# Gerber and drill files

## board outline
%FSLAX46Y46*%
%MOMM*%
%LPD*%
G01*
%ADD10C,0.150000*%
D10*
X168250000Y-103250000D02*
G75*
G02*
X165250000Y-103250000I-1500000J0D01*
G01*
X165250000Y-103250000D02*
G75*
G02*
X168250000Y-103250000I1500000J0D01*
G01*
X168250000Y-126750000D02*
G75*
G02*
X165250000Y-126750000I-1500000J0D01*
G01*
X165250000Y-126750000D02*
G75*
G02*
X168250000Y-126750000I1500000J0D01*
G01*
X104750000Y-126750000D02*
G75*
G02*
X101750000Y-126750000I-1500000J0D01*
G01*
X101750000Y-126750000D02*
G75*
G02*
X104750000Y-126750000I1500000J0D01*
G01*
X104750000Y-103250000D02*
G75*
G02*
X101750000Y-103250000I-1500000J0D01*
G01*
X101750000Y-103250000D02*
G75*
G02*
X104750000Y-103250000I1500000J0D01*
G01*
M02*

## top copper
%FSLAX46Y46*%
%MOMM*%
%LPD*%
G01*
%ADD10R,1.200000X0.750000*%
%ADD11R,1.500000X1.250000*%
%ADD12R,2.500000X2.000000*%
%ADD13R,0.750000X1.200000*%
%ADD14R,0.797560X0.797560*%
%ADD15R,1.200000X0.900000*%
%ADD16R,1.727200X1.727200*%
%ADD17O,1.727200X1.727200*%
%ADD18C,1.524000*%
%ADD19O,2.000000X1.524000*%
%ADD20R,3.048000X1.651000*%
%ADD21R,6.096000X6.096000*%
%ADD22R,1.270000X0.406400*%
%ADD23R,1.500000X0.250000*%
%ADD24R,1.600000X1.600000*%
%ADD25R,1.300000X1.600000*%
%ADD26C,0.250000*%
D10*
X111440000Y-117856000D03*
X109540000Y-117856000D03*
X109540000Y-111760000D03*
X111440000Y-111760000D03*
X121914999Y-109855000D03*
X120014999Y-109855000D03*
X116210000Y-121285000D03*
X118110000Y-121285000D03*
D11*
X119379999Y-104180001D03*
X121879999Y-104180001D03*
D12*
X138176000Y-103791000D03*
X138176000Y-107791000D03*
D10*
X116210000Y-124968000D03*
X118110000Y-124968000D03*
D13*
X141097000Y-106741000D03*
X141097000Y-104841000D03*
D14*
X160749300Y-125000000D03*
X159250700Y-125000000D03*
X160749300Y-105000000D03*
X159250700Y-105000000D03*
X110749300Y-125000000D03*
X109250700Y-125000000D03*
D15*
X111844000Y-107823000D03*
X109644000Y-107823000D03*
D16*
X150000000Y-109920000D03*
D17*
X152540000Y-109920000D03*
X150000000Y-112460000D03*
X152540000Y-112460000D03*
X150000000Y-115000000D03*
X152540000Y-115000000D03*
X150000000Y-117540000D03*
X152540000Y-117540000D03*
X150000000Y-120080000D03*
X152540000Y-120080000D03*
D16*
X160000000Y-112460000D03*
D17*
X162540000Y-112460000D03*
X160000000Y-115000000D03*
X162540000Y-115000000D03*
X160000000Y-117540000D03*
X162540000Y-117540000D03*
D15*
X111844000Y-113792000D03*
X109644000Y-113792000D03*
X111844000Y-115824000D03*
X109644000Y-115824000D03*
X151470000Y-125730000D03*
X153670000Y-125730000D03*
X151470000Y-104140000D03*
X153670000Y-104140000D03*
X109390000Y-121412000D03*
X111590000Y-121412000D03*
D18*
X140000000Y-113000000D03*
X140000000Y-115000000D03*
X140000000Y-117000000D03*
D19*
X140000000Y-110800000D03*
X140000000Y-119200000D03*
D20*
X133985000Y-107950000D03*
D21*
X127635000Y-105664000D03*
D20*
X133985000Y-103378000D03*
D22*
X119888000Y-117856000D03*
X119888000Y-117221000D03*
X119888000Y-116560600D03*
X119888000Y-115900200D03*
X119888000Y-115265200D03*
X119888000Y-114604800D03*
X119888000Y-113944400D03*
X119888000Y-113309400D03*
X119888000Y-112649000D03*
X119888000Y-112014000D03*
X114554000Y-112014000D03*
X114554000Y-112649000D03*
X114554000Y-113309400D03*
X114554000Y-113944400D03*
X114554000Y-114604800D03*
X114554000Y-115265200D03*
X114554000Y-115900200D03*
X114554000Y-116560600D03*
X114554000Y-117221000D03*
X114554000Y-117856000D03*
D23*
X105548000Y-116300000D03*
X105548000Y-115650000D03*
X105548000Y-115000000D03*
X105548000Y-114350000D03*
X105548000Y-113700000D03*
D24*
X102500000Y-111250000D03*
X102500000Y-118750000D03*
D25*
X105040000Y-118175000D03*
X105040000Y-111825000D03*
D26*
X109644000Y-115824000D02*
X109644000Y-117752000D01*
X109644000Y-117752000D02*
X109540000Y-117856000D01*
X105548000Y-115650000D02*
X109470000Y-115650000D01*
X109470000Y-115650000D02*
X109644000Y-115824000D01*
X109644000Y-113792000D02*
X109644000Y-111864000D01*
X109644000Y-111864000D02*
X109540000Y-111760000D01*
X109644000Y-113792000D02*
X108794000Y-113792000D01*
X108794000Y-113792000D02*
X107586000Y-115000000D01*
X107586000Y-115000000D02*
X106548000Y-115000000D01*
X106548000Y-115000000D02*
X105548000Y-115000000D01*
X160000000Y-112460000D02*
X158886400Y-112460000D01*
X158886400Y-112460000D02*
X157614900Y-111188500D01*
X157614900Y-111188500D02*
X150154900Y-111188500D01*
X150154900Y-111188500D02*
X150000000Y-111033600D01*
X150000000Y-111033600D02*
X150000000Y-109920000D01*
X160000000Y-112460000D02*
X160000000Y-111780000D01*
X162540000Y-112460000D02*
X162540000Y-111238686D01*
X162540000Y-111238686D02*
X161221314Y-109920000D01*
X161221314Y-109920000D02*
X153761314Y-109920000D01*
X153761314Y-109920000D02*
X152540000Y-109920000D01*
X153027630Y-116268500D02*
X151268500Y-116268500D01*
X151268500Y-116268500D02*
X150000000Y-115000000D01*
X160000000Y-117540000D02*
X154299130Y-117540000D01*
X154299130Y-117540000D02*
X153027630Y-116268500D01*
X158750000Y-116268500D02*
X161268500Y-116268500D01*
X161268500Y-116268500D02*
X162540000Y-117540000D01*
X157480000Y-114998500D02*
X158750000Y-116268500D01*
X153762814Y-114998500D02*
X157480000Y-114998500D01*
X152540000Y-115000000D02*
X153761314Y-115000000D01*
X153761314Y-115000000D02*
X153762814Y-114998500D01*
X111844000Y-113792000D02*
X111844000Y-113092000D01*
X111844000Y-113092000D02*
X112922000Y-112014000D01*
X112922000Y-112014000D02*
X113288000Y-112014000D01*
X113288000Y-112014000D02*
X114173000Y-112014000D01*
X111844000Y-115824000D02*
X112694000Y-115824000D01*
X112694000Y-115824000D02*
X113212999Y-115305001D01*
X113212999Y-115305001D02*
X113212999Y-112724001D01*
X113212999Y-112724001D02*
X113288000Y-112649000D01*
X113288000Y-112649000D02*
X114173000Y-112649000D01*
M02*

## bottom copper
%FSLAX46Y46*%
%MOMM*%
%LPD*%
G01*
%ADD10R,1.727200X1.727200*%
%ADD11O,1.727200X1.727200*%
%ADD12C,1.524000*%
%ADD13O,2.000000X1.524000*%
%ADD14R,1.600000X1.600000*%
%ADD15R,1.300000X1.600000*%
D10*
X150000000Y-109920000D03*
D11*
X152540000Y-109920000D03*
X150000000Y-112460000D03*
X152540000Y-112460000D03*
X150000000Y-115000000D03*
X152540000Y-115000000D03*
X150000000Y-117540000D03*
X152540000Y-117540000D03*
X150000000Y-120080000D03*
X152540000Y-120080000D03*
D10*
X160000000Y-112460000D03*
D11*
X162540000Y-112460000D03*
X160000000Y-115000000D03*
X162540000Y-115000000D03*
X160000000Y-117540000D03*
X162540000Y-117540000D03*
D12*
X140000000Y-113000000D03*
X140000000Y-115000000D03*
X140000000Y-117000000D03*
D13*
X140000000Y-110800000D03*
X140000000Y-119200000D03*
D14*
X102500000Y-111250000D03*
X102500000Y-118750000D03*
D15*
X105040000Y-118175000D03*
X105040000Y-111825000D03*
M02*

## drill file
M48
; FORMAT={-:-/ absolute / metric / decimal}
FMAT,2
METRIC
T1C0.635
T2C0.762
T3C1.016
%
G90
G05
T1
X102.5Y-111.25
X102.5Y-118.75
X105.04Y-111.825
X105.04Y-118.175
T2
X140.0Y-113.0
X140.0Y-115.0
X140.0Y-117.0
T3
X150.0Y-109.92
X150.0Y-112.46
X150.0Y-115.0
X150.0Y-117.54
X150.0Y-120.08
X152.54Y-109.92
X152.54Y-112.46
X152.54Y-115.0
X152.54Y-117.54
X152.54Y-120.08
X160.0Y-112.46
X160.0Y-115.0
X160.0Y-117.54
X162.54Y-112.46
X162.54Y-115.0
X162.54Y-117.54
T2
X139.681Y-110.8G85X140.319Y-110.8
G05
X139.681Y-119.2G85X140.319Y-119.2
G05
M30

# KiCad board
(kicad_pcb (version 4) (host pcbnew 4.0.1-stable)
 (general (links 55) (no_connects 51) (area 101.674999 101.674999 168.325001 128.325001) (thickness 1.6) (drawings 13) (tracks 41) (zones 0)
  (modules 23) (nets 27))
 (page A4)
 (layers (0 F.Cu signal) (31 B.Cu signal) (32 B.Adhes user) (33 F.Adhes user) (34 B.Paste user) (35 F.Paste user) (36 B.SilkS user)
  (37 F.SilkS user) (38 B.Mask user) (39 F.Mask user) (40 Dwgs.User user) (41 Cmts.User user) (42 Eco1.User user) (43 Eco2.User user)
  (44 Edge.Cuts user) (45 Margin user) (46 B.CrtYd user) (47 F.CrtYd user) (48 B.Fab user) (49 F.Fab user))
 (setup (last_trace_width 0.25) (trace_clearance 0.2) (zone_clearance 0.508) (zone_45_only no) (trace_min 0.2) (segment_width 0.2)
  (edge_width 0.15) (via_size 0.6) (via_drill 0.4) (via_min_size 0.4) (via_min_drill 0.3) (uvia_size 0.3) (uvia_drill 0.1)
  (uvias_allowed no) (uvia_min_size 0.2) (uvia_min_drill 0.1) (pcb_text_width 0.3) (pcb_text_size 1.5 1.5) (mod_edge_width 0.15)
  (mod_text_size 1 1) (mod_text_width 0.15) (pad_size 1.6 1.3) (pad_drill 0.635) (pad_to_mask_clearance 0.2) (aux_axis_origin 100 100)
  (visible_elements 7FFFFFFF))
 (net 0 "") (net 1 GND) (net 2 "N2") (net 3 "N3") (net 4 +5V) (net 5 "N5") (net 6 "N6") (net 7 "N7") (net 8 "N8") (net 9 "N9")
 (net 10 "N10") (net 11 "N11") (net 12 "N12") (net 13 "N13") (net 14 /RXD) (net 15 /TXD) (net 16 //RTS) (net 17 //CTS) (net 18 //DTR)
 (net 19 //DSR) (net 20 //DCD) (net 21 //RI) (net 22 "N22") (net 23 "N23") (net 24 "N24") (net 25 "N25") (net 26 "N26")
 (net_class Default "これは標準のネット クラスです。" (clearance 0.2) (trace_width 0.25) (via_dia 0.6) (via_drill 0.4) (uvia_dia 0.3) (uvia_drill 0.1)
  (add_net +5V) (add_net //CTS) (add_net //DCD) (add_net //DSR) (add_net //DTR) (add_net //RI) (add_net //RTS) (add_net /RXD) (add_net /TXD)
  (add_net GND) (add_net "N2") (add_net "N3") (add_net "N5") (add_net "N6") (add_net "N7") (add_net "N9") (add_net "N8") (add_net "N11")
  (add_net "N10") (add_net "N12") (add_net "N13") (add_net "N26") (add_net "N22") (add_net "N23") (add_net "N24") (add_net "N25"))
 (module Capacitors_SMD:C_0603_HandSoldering (layer F.Cu) (at 110.49 117.856 180)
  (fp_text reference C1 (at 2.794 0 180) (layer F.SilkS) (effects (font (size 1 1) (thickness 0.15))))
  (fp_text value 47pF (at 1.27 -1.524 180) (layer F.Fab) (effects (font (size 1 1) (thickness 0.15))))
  (pad 1 smd rect (at -0.95 0 180) (size 1.2 0.75) (layers F.Cu F.Paste F.Mask) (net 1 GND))
  (pad 2 smd rect (at 0.95 0 180) (size 1.2 0.75) (layers F.Cu F.Paste F.Mask) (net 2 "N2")))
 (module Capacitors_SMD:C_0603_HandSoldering (layer F.Cu) (at 110.49 111.76)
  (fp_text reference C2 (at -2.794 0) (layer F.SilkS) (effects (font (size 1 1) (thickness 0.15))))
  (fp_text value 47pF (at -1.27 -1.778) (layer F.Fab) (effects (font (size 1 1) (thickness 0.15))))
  (pad 1 smd rect (at -0.95 0) (size 1.2 0.75) (layers F.Cu F.Paste F.Mask) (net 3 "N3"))
  (pad 2 smd rect (at 0.95 0) (size 1.2 0.75) (layers F.Cu F.Paste F.Mask) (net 1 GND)))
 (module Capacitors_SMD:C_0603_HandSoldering (layer F.Cu) (at 120.964999 109.855 180)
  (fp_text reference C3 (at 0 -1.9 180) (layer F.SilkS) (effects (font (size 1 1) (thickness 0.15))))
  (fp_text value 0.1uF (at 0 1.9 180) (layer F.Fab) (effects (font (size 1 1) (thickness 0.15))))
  (pad 1 smd rect (at -0.95 0 180) (size 1.2 0.75) (layers F.Cu F.Paste F.Mask) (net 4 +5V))
  (pad 2 smd rect (at 0.95 0 180) (size 1.2 0.75) (layers F.Cu F.Paste F.Mask) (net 1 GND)))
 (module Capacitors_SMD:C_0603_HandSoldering (layer F.Cu) (at 117.16 121.285)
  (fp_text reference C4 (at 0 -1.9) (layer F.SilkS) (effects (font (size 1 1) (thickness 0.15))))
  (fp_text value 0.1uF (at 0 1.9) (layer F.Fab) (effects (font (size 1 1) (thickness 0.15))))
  (pad 1 smd rect (at -0.95 0) (size 1.2 0.75) (layers F.Cu F.Paste F.Mask) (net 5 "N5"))
  (pad 2 smd rect (at 0.95 0) (size 1.2 0.75) (layers F.Cu F.Paste F.Mask) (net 1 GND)))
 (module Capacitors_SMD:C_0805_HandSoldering (layer F.Cu) (at 120.629999 104.180001)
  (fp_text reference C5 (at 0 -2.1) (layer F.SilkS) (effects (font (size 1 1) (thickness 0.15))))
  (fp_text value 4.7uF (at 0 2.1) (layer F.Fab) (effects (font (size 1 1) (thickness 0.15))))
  (pad 1 smd rect (at -1.25 0) (size 1.5 1.25) (layers F.Cu F.Paste F.Mask) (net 1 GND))
  (pad 2 smd rect (at 1.25 0) (size 1.5 1.25) (layers F.Cu F.Paste F.Mask) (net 4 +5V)))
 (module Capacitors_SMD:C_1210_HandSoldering (layer F.Cu) (at 138.176 105.791 270)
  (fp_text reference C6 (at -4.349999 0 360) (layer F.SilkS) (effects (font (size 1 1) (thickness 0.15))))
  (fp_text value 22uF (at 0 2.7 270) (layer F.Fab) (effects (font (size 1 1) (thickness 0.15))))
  (pad 1 smd rect (at -2 0 270) (size 2 2.5) (layers F.Cu F.Paste F.Mask) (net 1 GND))
  (pad 2 smd rect (at 2 0 270) (size 2 2.5) (layers F.Cu F.Paste F.Mask) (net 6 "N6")))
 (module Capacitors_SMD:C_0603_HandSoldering (layer F.Cu) (at 117.16 124.968)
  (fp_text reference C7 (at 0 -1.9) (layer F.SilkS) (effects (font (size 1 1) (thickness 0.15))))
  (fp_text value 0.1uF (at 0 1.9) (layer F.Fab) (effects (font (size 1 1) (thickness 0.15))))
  (pad 1 smd rect (at -0.95 0) (size 1.2 0.75) (layers F.Cu F.Paste F.Mask) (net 6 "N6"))
  (pad 2 smd rect (at 0.95 0) (size 1.2 0.75) (layers F.Cu F.Paste F.Mask) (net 1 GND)))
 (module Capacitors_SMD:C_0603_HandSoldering (layer F.Cu) (at 141.097 105.791 90)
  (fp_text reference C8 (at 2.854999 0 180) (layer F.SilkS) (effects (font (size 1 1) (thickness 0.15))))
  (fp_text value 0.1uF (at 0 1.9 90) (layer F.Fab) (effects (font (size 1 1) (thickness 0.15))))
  (pad 1 smd rect (at -0.95 0 90) (size 1.2 0.75) (layers F.Cu F.Paste F.Mask) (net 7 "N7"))
  (pad 2 smd rect (at 0.95 0 90) (size 1.2 0.75) (layers F.Cu F.Paste F.Mask) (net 1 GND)))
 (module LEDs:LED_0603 (layer F.Cu) (at 160 125)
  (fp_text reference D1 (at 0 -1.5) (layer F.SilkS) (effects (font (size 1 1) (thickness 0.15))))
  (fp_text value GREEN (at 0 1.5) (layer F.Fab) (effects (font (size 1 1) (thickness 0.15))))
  (pad 2 smd rect (at 0.7493 0 180) (size 0.79756 0.79756) (layers F.Cu F.Paste F.Mask) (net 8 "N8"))
  (pad 1 smd rect (at -0.7493 0 180) (size 0.79756 0.79756) (layers F.Cu F.Paste F.Mask) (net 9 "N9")))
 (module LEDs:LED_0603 (layer F.Cu) (at 160 105)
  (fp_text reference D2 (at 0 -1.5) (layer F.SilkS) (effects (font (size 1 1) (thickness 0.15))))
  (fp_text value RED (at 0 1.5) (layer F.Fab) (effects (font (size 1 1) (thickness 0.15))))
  (pad 2 smd rect (at 0.7493 0 180) (size 0.79756 0.79756) (layers F.Cu F.Paste F.Mask) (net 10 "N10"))
  (pad 1 smd rect (at -0.7493 0 180) (size 0.79756 0.79756) (layers F.Cu F.Paste F.Mask) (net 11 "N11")))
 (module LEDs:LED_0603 (layer F.Cu) (at 110 125)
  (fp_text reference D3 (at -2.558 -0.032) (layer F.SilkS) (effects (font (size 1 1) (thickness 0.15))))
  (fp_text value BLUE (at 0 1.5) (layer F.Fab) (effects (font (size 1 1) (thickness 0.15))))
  (pad 2 smd rect (at 0.7493 0 180) (size 0.79756 0.79756) (layers F.Cu F.Paste F.Mask) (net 4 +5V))
  (pad 1 smd rect (at -0.7493 0 180) (size 0.79756 0.79756) (layers F.Cu F.Paste F.Mask) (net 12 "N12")))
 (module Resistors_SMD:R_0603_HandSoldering (layer F.Cu) (at 110.744 107.823 180)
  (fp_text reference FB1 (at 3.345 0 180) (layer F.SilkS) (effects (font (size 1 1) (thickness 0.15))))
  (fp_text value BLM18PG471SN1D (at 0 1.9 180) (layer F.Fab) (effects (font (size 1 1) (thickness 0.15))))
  (pad 1 smd rect (at -1.1 0 180) (size 1.2 0.9) (layers F.Cu F.Paste F.Mask) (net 4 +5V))
  (pad 2 smd rect (at 1.1 0 180) (size 1.2 0.9) (layers F.Cu F.Paste F.Mask) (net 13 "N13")))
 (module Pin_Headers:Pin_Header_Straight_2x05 (layer F.Cu) (at 150 109.92)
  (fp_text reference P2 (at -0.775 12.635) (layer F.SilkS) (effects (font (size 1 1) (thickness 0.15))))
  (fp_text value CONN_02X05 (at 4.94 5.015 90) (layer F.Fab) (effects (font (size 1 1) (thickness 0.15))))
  (pad 1 thru_hole rect (at 0 0) (size 1.7272 1.7272) (drill 1.016) (layers *.Cu *.Mask F.SilkS) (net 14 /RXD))
  (pad 2 thru_hole oval (at 2.54 0) (size 1.7272 1.7272) (drill 1.016) (layers *.Cu *.Mask F.SilkS) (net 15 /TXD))
  (pad 3 thru_hole oval (at 0 2.54) (size 1.7272 1.7272) (drill 1.016) (layers *.Cu *.Mask F.SilkS) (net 1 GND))
  (pad 4 thru_hole oval (at 2.54 2.54) (size 1.7272 1.7272) (drill 1.016) (layers *.Cu *.Mask F.SilkS) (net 7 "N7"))
  (pad 5 thru_hole oval (at 0 5.08) (size 1.7272 1.7272) (drill 1.016) (layers *.Cu *.Mask F.SilkS) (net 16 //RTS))
  (pad 6 thru_hole oval (at 2.54 5.08) (size 1.7272 1.7272) (drill 1.016) (layers *.Cu *.Mask F.SilkS) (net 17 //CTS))
  (pad 7 thru_hole oval (at 0 7.62) (size 1.7272 1.7272) (drill 1.016) (layers *.Cu *.Mask F.SilkS) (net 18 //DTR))
  (pad 8 thru_hole oval (at 2.54 7.62) (size 1.7272 1.7272) (drill 1.016) (layers *.Cu *.Mask F.SilkS) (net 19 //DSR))
  (pad 9 thru_hole oval (at 0 10.16) (size 1.7272 1.7272) (drill 1.016) (layers *.Cu *.Mask F.SilkS) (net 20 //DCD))
  (pad 10 thru_hole oval (at 2.54 10.16) (size 1.7272 1.7272) (drill 1.016) (layers *.Cu *.Mask F.SilkS) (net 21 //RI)))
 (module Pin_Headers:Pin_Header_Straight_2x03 (layer F.Cu) (at 160 112.46)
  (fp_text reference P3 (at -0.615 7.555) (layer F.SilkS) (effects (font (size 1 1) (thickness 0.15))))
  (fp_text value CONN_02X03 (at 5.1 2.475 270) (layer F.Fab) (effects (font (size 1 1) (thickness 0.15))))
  (pad 1 thru_hole rect (at 0 0) (size 1.7272 1.7272) (drill 1.016) (layers *.Cu *.Mask F.SilkS) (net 14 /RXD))
  (pad 2 thru_hole oval (at 2.54 0) (size 1.7272 1.7272) (drill 1.016) (layers *.Cu *.Mask F.SilkS) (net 15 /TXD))
  (pad 3 thru_hole oval (at 0 2.54) (size 1.7272 1.7272) (drill 1.016) (layers *.Cu *.Mask F.SilkS) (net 1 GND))
  (pad 4 thru_hole oval (at 2.54 2.54) (size 1.7272 1.7272) (drill 1.016) (layers *.Cu *.Mask F.SilkS) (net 7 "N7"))
  (pad 5 thru_hole oval (at 0 5.08) (size 1.7272 1.7272) (drill 1.016) (layers *.Cu *.Mask F.SilkS) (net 16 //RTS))
  (pad 6 thru_hole oval (at 2.54 5.08) (size 1.7272 1.7272) (drill 1.016) (layers *.Cu *.Mask F.SilkS) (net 17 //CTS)))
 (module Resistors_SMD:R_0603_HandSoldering (layer F.Cu) (at 110.744 113.792 180)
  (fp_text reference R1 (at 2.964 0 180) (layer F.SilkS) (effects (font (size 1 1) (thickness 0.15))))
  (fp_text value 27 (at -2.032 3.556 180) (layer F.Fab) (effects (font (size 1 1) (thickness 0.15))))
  (pad 1 smd rect (at -1.1 0 180) (size 1.2 0.9) (layers F.Cu F.Paste F.Mask) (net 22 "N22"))
  (pad 2 smd rect (at 1.1 0 180) (size 1.2 0.9) (layers F.Cu F.Paste F.Mask) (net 3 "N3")))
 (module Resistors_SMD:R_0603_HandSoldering (layer F.Cu) (at 110.744 115.824 180)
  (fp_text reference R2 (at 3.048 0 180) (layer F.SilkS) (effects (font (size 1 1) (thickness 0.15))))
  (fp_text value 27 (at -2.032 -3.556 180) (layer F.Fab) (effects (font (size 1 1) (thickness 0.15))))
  (pad 1 smd rect (at -1.1 0 180) (size 1.2 0.9) (layers F.Cu F.Paste F.Mask) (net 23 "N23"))
  (pad 2 smd rect (at 1.1 0 180) (size 1.2 0.9) (layers F.Cu F.Paste F.Mask) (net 2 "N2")))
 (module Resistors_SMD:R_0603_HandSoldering (layer F.Cu) (at 152.57 125.73)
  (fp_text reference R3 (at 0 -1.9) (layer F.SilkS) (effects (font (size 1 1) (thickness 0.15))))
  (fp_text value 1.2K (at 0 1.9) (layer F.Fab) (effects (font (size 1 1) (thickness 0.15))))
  (pad 1 smd rect (at -1.1 0) (size 1.2 0.9) (layers F.Cu F.Paste F.Mask) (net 4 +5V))
  (pad 2 smd rect (at 1.1 0) (size 1.2 0.9) (layers F.Cu F.Paste F.Mask) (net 8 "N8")))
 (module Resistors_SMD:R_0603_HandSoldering (layer F.Cu) (at 152.57 104.14)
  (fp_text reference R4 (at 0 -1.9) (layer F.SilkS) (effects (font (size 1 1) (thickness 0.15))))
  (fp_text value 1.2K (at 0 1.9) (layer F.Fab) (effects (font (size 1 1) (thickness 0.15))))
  (pad 1 smd rect (at -1.1 0) (size 1.2 0.9) (layers F.Cu F.Paste F.Mask) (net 4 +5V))
  (pad 2 smd rect (at 1.1 0) (size 1.2 0.9) (layers F.Cu F.Paste F.Mask) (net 10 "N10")))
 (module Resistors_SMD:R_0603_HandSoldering (layer F.Cu) (at 110.49 121.412)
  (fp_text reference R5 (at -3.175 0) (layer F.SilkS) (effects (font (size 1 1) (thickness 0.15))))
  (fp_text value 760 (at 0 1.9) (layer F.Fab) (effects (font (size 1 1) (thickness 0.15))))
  (pad 1 smd rect (at -1.1 0) (size 1.2 0.9) (layers F.Cu F.Paste F.Mask) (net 12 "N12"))
  (pad 2 smd rect (at 1.1 0) (size 1.2 0.9) (layers F.Cu F.Paste F.Mask) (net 1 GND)))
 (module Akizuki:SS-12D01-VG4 (layer F.Cu) (at 140 115 90)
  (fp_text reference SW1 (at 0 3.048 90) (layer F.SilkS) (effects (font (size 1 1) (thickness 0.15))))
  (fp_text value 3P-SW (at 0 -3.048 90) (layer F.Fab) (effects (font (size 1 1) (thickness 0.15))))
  (pad 3 thru_hole circle (at 2 0 90) (size 1.524 1.524) (drill 0.762) (layers *.Cu *.Mask F.SilkS) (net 4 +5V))
  (pad 2 thru_hole circle (at 0 0 90) (size 1.524 1.524) (drill 0.762) (layers *.Cu *.Mask F.SilkS) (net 7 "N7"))
  (pad 1 thru_hole circle (at -2 0 90) (size 1.524 1.524) (drill 0.762) (layers *.Cu *.Mask F.SilkS) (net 6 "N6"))
  (pad 0 thru_hole oval (at 4.2 0 90) (size 1.524 2) (drill oval 0.762 1.4) (layers *.Cu *.Mask F.SilkS))
  (pad 0 thru_hole oval (at -4.2 0 90) (size 1.524 2) (drill oval 0.762 1.4) (layers *.Cu *.Mask F.SilkS)))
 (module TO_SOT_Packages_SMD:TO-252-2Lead (layer F.Cu) (at 133.985 105.664 90)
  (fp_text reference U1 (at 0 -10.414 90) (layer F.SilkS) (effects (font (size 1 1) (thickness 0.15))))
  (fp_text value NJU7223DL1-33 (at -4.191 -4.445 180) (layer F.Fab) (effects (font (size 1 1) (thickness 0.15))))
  (pad 1 smd rect (at -2.286 0 90) (size 1.651 3.048) (layers F.Cu F.Paste F.Mask) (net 6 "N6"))
  (pad 2 smd rect (at 0 -6.35 90) (size 6.096 6.096) (layers F.Cu F.Paste F.Mask) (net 4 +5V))
  (pad 3 smd rect (at 2.286 0 90) (size 1.651 3.048) (layers F.Cu F.Paste F.Mask) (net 1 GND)))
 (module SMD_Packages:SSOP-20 (layer F.Cu) (at 117.221 114.935 90)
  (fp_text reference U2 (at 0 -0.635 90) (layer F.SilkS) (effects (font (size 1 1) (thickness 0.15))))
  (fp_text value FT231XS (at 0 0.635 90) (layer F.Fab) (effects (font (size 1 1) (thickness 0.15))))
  (pad 1 smd rect (at -2.921 2.667 90) (size 0.4064 1.27) (layers F.Cu F.Paste F.Mask) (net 18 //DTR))
  (pad 2 smd rect (at -2.286 2.667 90) (size 0.4064 1.27) (layers F.Cu F.Paste F.Mask) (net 16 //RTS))
  (pad 3 smd rect (at -1.6256 2.667 90) (size 0.4064 1.27) (layers F.Cu F.Paste F.Mask) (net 7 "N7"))
  (pad 4 smd rect (at -0.9652 2.667 90) (size 0.4064 1.27) (layers F.Cu F.Paste F.Mask) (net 14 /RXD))
  (pad 5 smd rect (at -0.3302 2.667 90) (size 0.4064 1.27) (layers F.Cu F.Paste F.Mask) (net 21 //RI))
  (pad 6 smd rect (at 0.3302 2.667 90) (size 0.4064 1.27) (layers F.Cu F.Paste F.Mask) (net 1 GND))
  (pad 7 smd rect (at 0.9906 2.667 90) (size 0.4064 1.27) (layers F.Cu F.Paste F.Mask) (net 19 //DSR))
  (pad 8 smd rect (at 1.6256 2.667 90) (size 0.4064 1.27) (layers F.Cu F.Paste F.Mask) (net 20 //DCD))
  (pad 9 smd rect (at 2.286 2.667 90) (size 0.4064 1.27) (layers F.Cu F.Paste F.Mask) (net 17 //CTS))
  (pad 10 smd rect (at 2.921 2.667 90) (size 0.4064 1.27) (layers F.Cu F.Paste F.Mask) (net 11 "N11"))
  (pad 11 smd rect (at 2.921 -2.667 90) (size 0.4064 1.27) (layers F.Cu F.Paste F.Mask) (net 22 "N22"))
  (pad 12 smd rect (at 2.286 -2.667 90) (size 0.4064 1.27) (layers F.Cu F.Paste F.Mask) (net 23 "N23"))
  (pad 13 smd rect (at 1.6256 -2.667 90) (size 0.4064 1.27) (layers F.Cu F.Paste F.Mask) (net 5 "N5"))
  (pad 14 smd rect (at 0.9906 -2.667 90) (size 0.4064 1.27) (layers F.Cu F.Paste F.Mask) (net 5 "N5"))
  (pad 15 smd rect (at 0.3302 -2.667 90) (size 0.4064 1.27) (layers F.Cu F.Paste F.Mask) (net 4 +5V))
  (pad 16 smd rect (at -0.3302 -2.667 90) (size 0.4064 1.27) (layers F.Cu F.Paste F.Mask) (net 1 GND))
  (pad 17 smd rect (at -0.9652 -2.667 90) (size 0.4064 1.27) (layers F.Cu F.Paste F.Mask) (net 9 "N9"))
  (pad 18 smd rect (at -1.6256 -2.667 90) (size 0.4064 1.27) (layers F.Cu F.Paste F.Mask) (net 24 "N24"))
  (pad 19 smd rect (at -2.286 -2.667 90) (size 0.4064 1.27) (layers F.Cu F.Paste F.Mask) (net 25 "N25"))
  (pad 20 smd rect (at -2.921 -2.667 90) (size 0.4064 1.27) (layers F.Cu F.Paste F.Mask) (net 15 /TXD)))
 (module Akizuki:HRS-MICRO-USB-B (layer F.Cu) (at 102.5 115 90)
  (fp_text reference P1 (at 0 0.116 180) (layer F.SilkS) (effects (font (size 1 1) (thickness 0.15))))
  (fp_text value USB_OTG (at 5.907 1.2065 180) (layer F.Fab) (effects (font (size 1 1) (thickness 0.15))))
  (pad 1 smd rect (at -1.3 3.048 90) (size 0.25 1.5) (layers F.Cu F.Paste F.Mask) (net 13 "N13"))
  (pad 2 smd rect (at -0.65 3.048 90) (size 0.25 1.5) (layers F.Cu F.Paste F.Mask) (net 2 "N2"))
  (pad 3 smd rect (at 0 3.048 90) (size 0.25 1.5) (layers F.Cu F.Paste F.Mask) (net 3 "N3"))
  (pad 4 smd rect (at 0.65 3.048 90) (size 0.25 1.5) (layers F.Cu F.Paste F.Mask) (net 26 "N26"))
  (pad 5 smd rect (at 1.3 3.048 90) (size 0.25 1.5) (layers F.Cu F.Paste F.Mask) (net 1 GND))
  (pad 0 thru_hole rect (at 3.75 0 90) (size 1.6 1.6) (drill 0.635) (layers *.Cu *.Mask F.SilkS))
  (pad 0 thru_hole rect (at -3.75 0 90) (size 1.6 1.6) (drill 0.635) (layers *.Cu *.Mask F.SilkS))
  (pad 0 thru_hole rect (at -3.175 2.54 90) (size 1.6 1.3) (drill 0.635) (layers *.Cu *.Mask F.SilkS))
  (pad 0 thru_hole rect (at 3.175 2.54 90) (size 1.6 1.3) (drill 0.635) (layers *.Cu *.Mask F.SilkS)))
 (gr_circle (center 166.75 103.25) (end 166.75 104.75) (layer Edge.Cuts) (width 0.15))
 (gr_circle (center 166.75 126.75) (end 166.75 125.25) (layer Edge.Cuts) (width 0.15))
 (gr_circle (center 103.25 126.75) (end 103.25 128.25) (layer Edge.Cuts) (width 0.15))
 (gr_circle (center 103.25 103.25) (end 103.25 101.75) (layer Edge.Cuts) (width 0.15))
 (segment (start 190.5 93.98) (end 194.31 93.98) (width 0.25) (layer Dwgs.User) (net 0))
 (segment (start 176.53 93.98) (end 190.5 93.98) (width 0.25) (layer Dwgs.User) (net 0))
 (segment (start 109.644 115.824) (end 109.644 117.752) (width 0.25) (layer F.Cu) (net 2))
 (segment (start 109.644 117.752) (end 109.54 117.856) (width 0.25) (layer F.Cu) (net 2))
 (segment (start 105.548 115.65) (end 109.47 115.65) (width 0.25) (layer F.Cu) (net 2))
 (segment (start 109.47 115.65) (end 109.644 115.824) (width 0.25) (layer F.Cu) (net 2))
 (segment (start 109.644 113.792) (end 109.644 111.864) (width 0.25) (layer F.Cu) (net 3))
 (segment (start 109.644 111.864) (end 109.54 111.76) (width 0.25) (layer F.Cu) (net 3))
 (segment (start 109.644 113.792) (end 108.794 113.792) (width 0.25) (layer F.Cu) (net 3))
 (segment (start 108.794 113.792) (end 107.586 115) (width 0.25) (layer F.Cu) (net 3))
 (segment (start 107.586 115) (end 106.548 115) (width 0.25) (layer F.Cu) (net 3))
 (segment (start 106.548 115) (end 105.548 115) (width 0.25) (layer F.Cu) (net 3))
 (segment (start 160 112.46) (end 158.8864 112.46) (width 0.25) (layer F.Cu) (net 14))
 (segment (start 158.8864 112.46) (end 157.6149 111.1885) (width 0.25) (layer F.Cu) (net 14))
 (segment (start 157.6149 111.1885) (end 150.1549 111.1885) (width 0.25) (layer F.Cu) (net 14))
 (segment (start 150.1549 111.1885) (end 150 111.0336) (width 0.25) (layer F.Cu) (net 14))
 (segment (start 150 111.0336) (end 150 109.92) (width 0.25) (layer F.Cu) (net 14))
 (segment (start 160 112.46) (end 160 111.78) (width 0.25) (layer F.Cu) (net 14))
 (segment (start 162.54 112.46) (end 162.54 111.238686) (width 0.25) (layer F.Cu) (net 15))
 (segment (start 162.54 111.238686) (end 161.221314 109.92) (width 0.25) (layer F.Cu) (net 15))
 (segment (start 161.221314 109.92) (end 153.761314 109.92) (width 0.25) (layer F.Cu) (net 15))
 (segment (start 153.761314 109.92) (end 152.54 109.92) (width 0.25) (layer F.Cu) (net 15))
 (segment (start 153.02763 116.2685) (end 151.2685 116.2685) (width 0.25) (layer F.Cu) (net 16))
 (segment (start 151.2685 116.2685) (end 150 115) (width 0.25) (layer F.Cu) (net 16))
 (segment (start 160 117.54) (end 154.29913 117.54) (width 0.25) (layer F.Cu) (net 16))
 (segment (start 154.29913 117.54) (end 153.02763 116.2685) (width 0.25) (layer F.Cu) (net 16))
 (segment (start 158.75 116.2685) (end 161.2685 116.2685) (width 0.25) (layer F.Cu) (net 17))
 (segment (start 161.2685 116.2685) (end 162.54 117.54) (width 0.25) (layer F.Cu) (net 17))
 (segment (start 157.48 114.9985) (end 158.75 116.2685) (width 0.25) (layer F.Cu) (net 17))
 (segment (start 153.762814 114.9985) (end 157.48 114.9985) (width 0.25) (layer F.Cu) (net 17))
 (segment (start 152.54 115) (end 153.761314 115) (width 0.25) (layer F.Cu) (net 17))
 (segment (start 153.761314 115) (end 153.762814 114.9985) (width 0.25) (layer F.Cu) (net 17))
 (segment (start 111.844 113.792) (end 111.844 113.092) (width 0.25) (layer F.Cu) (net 22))
 (segment (start 111.844 113.092) (end 112.922 112.014) (width 0.25) (layer F.Cu) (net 22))
 (segment (start 112.922 112.014) (end 113.288 112.014) (width 0.25) (layer F.Cu) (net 22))
 (segment (start 113.288 112.014) (end 114.173 112.014) (width 0.25) (layer F.Cu) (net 22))
 (segment (start 111.844 115.824) (end 112.694 115.824) (width 0.25) (layer F.Cu) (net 23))
 (segment (start 112.694 115.824) (end 113.212999 115.305001) (width 0.25) (layer F.Cu) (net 23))
 (segment (start 113.212999 115.305001) (end 113.212999 112.724001) (width 0.25) (layer F.Cu) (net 23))
 (segment (start 113.212999 112.724001) (end 113.288 112.649) (width 0.25) (layer F.Cu) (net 23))
 (segment (start 113.288 112.649) (end 114.173 112.649) (width 0.25) (layer F.Cu) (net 23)))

